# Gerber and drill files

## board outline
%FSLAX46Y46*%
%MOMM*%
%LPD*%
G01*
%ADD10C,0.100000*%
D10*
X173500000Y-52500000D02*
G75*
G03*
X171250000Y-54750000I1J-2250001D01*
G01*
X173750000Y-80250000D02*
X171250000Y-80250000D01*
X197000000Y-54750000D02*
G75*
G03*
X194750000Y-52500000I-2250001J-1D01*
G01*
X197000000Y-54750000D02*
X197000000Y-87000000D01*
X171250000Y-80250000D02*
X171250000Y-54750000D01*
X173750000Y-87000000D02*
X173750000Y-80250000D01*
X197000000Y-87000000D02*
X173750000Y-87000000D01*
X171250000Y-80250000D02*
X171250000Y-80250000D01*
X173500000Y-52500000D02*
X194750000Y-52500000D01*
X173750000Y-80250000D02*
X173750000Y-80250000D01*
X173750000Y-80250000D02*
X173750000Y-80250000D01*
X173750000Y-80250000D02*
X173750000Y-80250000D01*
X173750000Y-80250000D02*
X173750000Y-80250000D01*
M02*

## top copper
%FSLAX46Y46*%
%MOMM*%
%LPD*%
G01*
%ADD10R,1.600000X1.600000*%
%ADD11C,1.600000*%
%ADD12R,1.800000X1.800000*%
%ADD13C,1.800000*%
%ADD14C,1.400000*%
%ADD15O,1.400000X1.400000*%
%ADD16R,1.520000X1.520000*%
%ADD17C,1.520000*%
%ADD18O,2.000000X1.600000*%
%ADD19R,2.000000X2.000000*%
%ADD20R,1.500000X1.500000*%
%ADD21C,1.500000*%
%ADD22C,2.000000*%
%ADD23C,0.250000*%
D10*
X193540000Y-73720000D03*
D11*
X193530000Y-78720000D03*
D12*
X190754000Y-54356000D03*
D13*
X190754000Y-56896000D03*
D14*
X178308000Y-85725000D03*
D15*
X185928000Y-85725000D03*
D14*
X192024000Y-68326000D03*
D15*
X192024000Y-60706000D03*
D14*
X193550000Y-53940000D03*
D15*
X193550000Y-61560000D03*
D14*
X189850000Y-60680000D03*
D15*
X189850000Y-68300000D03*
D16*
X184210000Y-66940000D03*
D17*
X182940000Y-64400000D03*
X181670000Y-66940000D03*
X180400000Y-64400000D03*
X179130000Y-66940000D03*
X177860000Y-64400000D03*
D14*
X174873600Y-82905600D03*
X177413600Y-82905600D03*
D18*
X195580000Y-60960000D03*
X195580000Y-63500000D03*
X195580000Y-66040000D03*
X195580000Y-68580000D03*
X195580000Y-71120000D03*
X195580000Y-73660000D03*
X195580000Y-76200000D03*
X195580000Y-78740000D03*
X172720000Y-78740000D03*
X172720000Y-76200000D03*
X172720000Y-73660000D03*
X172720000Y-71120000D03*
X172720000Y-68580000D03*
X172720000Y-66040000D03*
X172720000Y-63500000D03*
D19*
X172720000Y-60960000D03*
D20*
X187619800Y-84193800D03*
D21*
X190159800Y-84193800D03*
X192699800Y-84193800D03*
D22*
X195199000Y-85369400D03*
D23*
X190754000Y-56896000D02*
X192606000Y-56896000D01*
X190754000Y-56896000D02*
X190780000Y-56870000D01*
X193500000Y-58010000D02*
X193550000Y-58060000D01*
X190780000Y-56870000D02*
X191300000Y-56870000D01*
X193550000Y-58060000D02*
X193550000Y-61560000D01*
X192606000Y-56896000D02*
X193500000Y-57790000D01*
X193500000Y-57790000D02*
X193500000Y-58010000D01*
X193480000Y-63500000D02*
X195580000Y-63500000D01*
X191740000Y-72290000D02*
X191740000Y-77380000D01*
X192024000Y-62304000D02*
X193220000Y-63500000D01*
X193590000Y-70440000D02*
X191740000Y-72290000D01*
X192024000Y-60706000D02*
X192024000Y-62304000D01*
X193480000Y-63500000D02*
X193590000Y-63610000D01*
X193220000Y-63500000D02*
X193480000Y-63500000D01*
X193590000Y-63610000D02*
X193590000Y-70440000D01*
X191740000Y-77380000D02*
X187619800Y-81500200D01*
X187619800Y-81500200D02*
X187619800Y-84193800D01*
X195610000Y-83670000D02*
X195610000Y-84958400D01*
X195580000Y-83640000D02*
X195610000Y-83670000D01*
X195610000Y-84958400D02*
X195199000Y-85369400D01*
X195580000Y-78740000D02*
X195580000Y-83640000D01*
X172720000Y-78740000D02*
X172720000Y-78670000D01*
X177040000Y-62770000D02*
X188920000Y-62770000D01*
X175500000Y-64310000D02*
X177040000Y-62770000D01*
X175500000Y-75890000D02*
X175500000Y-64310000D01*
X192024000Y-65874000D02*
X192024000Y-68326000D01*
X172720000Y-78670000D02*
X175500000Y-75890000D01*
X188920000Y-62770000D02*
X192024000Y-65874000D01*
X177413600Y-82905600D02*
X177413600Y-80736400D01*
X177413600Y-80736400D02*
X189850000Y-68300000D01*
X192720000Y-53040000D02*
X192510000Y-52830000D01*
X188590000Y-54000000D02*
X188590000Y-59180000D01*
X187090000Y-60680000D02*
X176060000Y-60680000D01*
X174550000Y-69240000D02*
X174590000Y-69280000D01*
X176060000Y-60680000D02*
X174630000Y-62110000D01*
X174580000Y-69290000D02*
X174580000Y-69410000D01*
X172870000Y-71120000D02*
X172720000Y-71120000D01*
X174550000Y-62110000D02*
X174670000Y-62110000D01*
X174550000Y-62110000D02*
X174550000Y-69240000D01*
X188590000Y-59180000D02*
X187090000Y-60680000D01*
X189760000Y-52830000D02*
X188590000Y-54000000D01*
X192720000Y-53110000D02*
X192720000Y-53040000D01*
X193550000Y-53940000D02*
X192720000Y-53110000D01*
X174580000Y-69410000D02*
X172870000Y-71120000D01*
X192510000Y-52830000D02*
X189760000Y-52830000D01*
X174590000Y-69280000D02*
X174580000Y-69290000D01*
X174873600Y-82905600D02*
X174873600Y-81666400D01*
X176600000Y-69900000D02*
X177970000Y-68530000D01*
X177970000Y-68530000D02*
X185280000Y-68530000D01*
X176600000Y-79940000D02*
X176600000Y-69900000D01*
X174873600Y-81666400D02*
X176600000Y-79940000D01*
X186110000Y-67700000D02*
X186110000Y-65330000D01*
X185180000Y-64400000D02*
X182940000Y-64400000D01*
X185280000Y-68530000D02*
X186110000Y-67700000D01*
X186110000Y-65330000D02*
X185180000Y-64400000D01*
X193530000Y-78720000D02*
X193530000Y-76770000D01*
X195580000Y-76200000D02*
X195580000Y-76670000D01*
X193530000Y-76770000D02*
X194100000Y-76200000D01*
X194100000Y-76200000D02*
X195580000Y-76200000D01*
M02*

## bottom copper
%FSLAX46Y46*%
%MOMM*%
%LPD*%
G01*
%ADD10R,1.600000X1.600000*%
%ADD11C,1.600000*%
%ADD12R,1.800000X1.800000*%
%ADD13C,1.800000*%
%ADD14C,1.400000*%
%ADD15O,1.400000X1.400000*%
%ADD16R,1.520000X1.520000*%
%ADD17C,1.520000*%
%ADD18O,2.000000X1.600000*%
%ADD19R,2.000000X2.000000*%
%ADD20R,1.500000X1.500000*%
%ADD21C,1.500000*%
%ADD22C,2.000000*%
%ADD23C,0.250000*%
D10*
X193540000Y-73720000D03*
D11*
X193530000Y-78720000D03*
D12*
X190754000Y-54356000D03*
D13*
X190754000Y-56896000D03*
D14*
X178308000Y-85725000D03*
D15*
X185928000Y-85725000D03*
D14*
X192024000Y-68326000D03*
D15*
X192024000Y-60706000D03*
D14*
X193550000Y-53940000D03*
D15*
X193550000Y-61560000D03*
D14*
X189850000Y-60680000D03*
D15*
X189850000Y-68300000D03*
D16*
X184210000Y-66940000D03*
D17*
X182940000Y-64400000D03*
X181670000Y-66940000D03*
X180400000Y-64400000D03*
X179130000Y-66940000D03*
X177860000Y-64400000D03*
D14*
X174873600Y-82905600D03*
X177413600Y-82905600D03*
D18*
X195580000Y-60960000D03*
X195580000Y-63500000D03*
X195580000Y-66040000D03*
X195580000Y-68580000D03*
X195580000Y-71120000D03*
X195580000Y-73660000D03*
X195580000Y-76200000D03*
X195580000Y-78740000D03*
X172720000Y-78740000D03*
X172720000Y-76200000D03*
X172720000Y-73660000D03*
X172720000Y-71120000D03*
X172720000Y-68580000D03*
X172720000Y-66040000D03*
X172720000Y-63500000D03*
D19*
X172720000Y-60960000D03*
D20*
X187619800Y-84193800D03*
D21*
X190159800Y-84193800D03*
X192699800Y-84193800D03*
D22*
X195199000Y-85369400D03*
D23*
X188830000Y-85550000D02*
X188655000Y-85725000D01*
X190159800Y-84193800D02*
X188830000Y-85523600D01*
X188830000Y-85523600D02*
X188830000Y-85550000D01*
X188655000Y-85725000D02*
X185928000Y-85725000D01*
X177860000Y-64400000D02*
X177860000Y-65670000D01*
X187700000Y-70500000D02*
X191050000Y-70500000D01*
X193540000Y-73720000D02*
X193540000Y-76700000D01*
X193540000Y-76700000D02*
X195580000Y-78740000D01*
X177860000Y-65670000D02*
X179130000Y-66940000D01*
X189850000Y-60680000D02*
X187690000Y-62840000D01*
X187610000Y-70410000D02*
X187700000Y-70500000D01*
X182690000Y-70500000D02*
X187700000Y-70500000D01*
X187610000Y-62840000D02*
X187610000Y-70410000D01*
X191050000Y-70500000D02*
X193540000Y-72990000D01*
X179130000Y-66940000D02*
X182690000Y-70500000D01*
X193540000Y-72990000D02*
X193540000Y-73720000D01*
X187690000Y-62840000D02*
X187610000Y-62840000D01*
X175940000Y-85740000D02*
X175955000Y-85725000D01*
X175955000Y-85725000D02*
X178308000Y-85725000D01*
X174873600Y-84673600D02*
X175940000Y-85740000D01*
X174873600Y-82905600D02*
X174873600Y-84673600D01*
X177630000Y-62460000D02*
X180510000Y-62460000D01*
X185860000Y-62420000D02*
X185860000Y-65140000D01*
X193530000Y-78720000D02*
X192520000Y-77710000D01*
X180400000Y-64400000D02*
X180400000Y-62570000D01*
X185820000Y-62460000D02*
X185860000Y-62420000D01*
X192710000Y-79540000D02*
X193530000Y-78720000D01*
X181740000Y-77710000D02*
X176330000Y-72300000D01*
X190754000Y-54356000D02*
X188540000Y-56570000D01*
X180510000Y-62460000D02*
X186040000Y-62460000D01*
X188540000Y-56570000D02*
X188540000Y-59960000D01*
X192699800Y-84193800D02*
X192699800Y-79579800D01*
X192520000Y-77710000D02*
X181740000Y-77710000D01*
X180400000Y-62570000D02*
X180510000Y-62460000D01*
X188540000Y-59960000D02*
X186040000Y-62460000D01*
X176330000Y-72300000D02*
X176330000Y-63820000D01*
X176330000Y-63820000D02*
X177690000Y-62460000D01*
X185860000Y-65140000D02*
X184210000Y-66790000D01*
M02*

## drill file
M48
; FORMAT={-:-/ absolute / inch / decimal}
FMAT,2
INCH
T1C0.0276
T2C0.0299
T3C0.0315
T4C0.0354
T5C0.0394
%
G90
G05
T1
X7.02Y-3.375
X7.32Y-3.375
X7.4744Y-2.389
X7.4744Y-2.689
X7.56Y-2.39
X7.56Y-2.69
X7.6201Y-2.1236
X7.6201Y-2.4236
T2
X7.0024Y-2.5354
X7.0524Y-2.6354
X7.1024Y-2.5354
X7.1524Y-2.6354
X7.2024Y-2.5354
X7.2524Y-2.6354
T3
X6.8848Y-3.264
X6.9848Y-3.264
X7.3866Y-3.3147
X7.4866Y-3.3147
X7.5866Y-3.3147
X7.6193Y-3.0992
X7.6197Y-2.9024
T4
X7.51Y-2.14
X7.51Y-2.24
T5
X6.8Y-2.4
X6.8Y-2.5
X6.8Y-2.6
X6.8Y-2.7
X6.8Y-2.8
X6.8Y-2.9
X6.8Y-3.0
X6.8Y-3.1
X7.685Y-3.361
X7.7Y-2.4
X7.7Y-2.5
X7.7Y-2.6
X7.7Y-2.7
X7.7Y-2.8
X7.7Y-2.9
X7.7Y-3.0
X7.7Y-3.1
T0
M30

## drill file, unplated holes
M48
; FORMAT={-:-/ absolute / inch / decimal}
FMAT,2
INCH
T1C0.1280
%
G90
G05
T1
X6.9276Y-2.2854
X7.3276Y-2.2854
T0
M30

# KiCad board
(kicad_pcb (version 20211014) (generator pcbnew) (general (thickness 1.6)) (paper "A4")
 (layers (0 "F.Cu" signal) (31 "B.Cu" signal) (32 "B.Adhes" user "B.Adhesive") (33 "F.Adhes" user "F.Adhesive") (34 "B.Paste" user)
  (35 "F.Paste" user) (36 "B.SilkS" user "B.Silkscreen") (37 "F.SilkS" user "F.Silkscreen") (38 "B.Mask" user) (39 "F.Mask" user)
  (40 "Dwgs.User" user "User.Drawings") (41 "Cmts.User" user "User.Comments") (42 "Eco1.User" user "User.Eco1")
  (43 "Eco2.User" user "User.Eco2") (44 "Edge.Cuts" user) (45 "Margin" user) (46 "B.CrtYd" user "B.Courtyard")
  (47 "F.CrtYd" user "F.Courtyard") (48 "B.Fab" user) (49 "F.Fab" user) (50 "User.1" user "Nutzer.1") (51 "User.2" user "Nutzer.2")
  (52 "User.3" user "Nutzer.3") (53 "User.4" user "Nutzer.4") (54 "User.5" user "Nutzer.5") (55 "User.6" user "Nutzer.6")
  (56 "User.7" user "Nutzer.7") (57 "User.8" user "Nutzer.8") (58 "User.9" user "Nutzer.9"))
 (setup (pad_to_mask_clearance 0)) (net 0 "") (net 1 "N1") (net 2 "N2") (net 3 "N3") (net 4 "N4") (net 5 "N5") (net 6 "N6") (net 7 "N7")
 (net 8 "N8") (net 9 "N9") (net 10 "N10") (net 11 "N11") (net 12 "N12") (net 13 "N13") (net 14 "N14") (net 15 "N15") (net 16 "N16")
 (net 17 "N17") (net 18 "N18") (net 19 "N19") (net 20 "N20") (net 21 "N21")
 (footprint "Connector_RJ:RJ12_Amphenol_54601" (layer "F.Cu") (at 184.21 66.94 180)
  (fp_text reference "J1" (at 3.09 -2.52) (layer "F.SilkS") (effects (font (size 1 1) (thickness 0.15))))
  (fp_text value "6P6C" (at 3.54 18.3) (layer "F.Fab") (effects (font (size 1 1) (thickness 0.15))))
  (pad "" np_thru_hole circle (at -1.91 8.89 180) (size 3.25 3.25) (drill 3.25) (layers *.Cu *.Mask))
  (pad "" np_thru_hole circle (at 8.25 8.89 180) (size 3.25 3.25) (drill 3.25) (layers *.Cu *.Mask))
  (pad "1" thru_hole rect (at 0 0 180) (size 1.52 1.52) (drill 0.76) (layers *.Cu *.Mask) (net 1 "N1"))
  (pad "2" thru_hole circle (at 1.27 2.54 180) (size 1.52 1.52) (drill 0.76) (layers *.Cu *.Mask) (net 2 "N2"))
  (pad "3" thru_hole circle (at 2.54 0 180) (size 1.52 1.52) (drill 0.76) (layers *.Cu *.Mask) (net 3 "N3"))
  (pad "4" thru_hole circle (at 3.81 2.54 180) (size 1.52 1.52) (drill 0.76) (layers *.Cu *.Mask) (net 1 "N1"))
  (pad "5" thru_hole circle (at 5.08 0 180) (size 1.52 1.52) (drill 0.76) (layers *.Cu *.Mask) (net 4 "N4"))
  (pad "6" thru_hole circle (at 6.35 2.54 180) (size 1.52 1.52) (drill 0.76) (layers *.Cu *.Mask) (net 4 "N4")))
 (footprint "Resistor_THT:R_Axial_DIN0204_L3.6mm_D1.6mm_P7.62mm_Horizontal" (layer "F.Cu") (at 192.024 68.326 90)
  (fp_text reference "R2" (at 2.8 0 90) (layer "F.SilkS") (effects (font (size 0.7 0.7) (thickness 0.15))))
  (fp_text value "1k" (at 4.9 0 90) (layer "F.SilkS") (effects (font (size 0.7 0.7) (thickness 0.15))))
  (pad "1" thru_hole circle (at 0 0 90) (size 1.4 1.4) (drill 0.7) (layers *.Cu *.Mask) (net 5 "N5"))
  (pad "2" thru_hole oval (at 7.62 0 90) (size 1.4 1.4) (drill 0.7) (layers *.Cu *.Mask) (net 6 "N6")))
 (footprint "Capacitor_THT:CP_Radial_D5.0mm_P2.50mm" (layer "F.Cu") (at 193.6 74.94 -90)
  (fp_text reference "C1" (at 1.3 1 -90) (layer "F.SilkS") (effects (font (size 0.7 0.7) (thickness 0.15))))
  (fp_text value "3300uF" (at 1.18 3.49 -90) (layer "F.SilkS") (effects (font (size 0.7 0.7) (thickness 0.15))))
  (pad "1" thru_hole rect (at -1.22 0.06 270) (size 1.6 1.6) (drill 0.8) (layers *.Cu *.Mask) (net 4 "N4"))
  (pad "2" thru_hole circle (at 3.78 0.07 270) (size 1.6 1.6) (drill 0.8) (layers *.Cu *.Mask) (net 1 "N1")))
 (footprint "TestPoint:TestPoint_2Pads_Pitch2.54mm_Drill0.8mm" (layer "F.Cu") (at 174.8736 82.9056)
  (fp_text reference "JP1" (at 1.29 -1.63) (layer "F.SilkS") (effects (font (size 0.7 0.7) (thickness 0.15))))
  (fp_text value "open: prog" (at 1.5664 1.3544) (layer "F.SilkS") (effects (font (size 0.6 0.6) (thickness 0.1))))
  (pad "1" thru_hole circle (at 0 0) (size 1.4 1.4) (drill 0.8) (layers *.Cu *.Mask) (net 2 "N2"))
  (pad "2" thru_hole circle (at 2.54 0) (size 1.4 1.4) (drill 0.8) (layers *.Cu *.Mask) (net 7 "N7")))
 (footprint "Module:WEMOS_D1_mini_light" (layer "F.Cu") (at 172.72 60.96)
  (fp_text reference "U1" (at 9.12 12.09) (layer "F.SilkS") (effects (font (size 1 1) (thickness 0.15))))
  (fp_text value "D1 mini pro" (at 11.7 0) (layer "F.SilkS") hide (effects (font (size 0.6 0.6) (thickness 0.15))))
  (pad "1" thru_hole rect (at 0 0) (size 2 2) (drill 1) (layers *.Cu *.Mask) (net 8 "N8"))
  (pad "2" thru_hole oval (at 0 2.54) (size 2 1.6) (drill 1) (layers *.Cu *.Mask) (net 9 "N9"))
  (pad "3" thru_hole oval (at 0 5.08) (size 2 1.6) (drill 1) (layers *.Cu *.Mask) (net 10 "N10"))
  (pad "4" thru_hole oval (at 0 7.62) (size 2 1.6) (drill 1) (layers *.Cu *.Mask) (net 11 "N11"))
  (pad "5" thru_hole oval (at 0 10.16) (size 2 1.6) (drill 1) (layers *.Cu *.Mask) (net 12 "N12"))
  (pad "6" thru_hole oval (at 0 12.7) (size 2 1.6) (drill 1) (layers *.Cu *.Mask) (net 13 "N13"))
  (pad "7" thru_hole oval (at 0 15.24) (size 2 1.6) (drill 1) (layers *.Cu *.Mask) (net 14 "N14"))
  (pad "8" thru_hole oval (at 0 17.78) (size 2 1.6) (drill 1) (layers *.Cu *.Mask) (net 5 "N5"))
  (pad "9" thru_hole oval (at 22.86 17.78) (size 2 1.6) (drill 1) (layers *.Cu *.Mask) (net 4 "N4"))
  (pad "10" thru_hole oval (at 22.86 15.24) (size 2 1.6) (drill 1) (layers *.Cu *.Mask) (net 1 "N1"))
  (pad "11" thru_hole oval (at 22.86 12.7) (size 2 1.6) (drill 1) (layers *.Cu *.Mask) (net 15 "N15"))
  (pad "12" thru_hole oval (at 22.86 10.16) (size 2 1.6) (drill 1) (layers *.Cu *.Mask) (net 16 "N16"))
  (pad "13" thru_hole oval (at 22.86 7.62) (size 2 1.6) (drill 1) (layers *.Cu *.Mask) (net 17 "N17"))
  (pad "14" thru_hole oval (at 22.86 5.08) (size 2 1.6) (drill 1) (layers *.Cu *.Mask) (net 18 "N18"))
  (pad "15" thru_hole oval (at 22.86 2.54) (size 2 1.6) (drill 1) (layers *.Cu *.Mask) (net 6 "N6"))
  (pad "16" thru_hole oval (at 22.86 0) (size 2 1.6) (drill 1) (layers *.Cu *.Mask) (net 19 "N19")))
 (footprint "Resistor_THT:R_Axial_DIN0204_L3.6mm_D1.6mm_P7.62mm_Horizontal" (layer "F.Cu") (at 193.55 53.94 -90)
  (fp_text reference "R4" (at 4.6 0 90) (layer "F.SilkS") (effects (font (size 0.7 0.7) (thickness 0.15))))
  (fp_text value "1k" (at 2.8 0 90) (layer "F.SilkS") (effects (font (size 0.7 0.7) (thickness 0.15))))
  (pad "1" thru_hole circle (at 0 0 270) (size 1.4 1.4) (drill 0.7) (layers *.Cu *.Mask) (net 12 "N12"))
  (pad "2" thru_hole oval (at 7.62 0 270) (size 1.4 1.4) (drill 0.7) (layers *.Cu *.Mask) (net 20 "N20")))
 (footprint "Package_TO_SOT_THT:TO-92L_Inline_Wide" (layer "F.Cu") (at 187.6198 84.1938)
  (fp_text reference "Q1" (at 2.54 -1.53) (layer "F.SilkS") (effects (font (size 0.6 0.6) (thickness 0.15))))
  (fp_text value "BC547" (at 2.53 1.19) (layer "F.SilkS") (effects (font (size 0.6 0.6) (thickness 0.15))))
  (pad "1" thru_hole rect (at 0 0) (size 1.5 1.5) (drill 0.8) (layers *.Cu *.Mask) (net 6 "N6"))
  (pad "2" thru_hole circle (at 2.54 0) (size 1.5 1.5) (drill 0.8) (layers *.Cu *.Mask) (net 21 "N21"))
  (pad "3" thru_hole circle (at 5.08 0) (size 1.5 1.5) (drill 0.8) (layers *.Cu *.Mask) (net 1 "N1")))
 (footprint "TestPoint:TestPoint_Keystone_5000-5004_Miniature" (layer "F.Cu") (at 195.199 85.3694)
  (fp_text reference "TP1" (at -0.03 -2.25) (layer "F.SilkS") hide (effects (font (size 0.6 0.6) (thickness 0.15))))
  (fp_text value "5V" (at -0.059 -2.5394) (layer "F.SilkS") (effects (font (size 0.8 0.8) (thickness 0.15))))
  (pad "1" thru_hole circle (at 0 0) (size 2 2) (drill 1) (layers *.Cu *.Mask) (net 4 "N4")))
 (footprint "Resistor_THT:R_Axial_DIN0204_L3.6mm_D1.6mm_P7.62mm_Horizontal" (layer "F.Cu") (at 189.85 60.68 -90)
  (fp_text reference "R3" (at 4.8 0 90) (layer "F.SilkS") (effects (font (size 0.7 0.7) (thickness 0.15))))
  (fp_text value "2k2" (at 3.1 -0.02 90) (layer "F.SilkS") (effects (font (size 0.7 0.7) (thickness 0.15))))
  (pad "1" thru_hole circle (at 0 0 270) (size 1.4 1.4) (drill 0.7) (layers *.Cu *.Mask) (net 4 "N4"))
  (pad "2" thru_hole oval (at 7.62 0 270) (size 1.4 1.4) (drill 0.7) (layers *.Cu *.Mask) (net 7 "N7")))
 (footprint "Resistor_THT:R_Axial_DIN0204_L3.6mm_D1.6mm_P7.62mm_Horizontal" (layer "F.Cu") (at 178.308 85.725)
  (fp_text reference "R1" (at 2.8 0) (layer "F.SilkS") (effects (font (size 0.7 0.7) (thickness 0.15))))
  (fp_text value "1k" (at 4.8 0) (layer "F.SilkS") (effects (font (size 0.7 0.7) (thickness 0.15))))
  (pad "1" thru_hole circle (at 0 0) (size 1.4 1.4) (drill 0.7) (layers *.Cu *.Mask) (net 2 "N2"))
  (pad "2" thru_hole oval (at 7.62 0) (size 1.4 1.4) (drill 0.7) (layers *.Cu *.Mask) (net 21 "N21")))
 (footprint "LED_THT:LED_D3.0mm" (layer "F.Cu") (at 190.754 54.356 -90)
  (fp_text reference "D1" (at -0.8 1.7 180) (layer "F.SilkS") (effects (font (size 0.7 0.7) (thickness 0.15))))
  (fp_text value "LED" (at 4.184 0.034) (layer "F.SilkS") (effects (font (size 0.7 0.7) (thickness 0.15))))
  (pad "1" thru_hole rect (at 0 0 270) (size 1.8 1.8) (drill 0.9) (layers *.Cu *.Mask) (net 1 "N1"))
  (pad "2" thru_hole circle (at 2.54 0 270) (size 1.8 1.8) (drill 0.9) (layers *.Cu *.Mask) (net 20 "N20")))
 (gr_arc (start 171.25 54.75) (mid 171.90901 53.15901) (end 173.5 52.5) (layer "Edge.Cuts") (width 0.1))
 (gr_line (start 173.75 80.25) (end 171.25 80.25) (layer "Edge.Cuts") (width 0.1))
 (gr_arc (start 194.75 52.5) (mid 196.34099 53.15901) (end 197 54.75) (layer "Edge.Cuts") (width 0.1))
 (gr_line (start 197 54.75) (end 197 87) (layer "Edge.Cuts") (width 0.1))
 (gr_line (start 171.25 80.25) (end 171.25 54.75) (layer "Edge.Cuts") (width 0.1))
 (gr_line (start 173.75 87) (end 173.75 80.25) (layer "Edge.Cuts") (width 0.1))
 (gr_line (start 197 87) (end 173.75 87) (layer "Edge.Cuts") (width 0.1))
 (gr_line (start 171.25 80.25) (end 171.25 80.25) (layer "Edge.Cuts") (width 0.1))
 (gr_line (start 173.5 52.5) (end 194.75 52.5) (layer "Edge.Cuts") (width 0.1))
 (gr_rect (start 173.75 80.25) (end 173.75 80.25) (layer "Edge.Cuts") (width 0.1) (fill none))
 (segment (start 190.754 56.896) (end 192.606 56.896) (width 0.25) (layer "F.Cu") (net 20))
 (segment (start 190.754 56.896) (end 190.78 56.87) (width 0.25) (layer "F.Cu") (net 20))
 (segment (start 193.5 58.01) (end 193.55 58.06) (width 0.25) (layer "F.Cu") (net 20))
 (segment (start 190.78 56.87) (end 191.3 56.87) (width 0.25) (layer "F.Cu") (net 20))
 (segment (start 193.55 58.06) (end 193.55 61.56) (width 0.25) (layer "F.Cu") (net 20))
 (segment (start 192.606 56.896) (end 193.5 57.79) (width 0.25) (layer "F.Cu") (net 20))
 (segment (start 193.5 57.79) (end 193.5 58.01) (width 0.25) (layer "F.Cu") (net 20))
 (segment (start 188.83 85.55) (end 188.655 85.725) (width 0.25) (layer "B.Cu") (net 21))
 (segment (start 190.1598 84.1938) (end 188.83 85.5236) (width 0.25) (layer "B.Cu") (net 21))
 (segment (start 188.83 85.5236) (end 188.83 85.55) (width 0.25) (layer "B.Cu") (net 21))
 (segment (start 188.655 85.725) (end 185.928 85.725) (width 0.25) (layer "B.Cu") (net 21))
 (segment (start 193.48 63.5) (end 195.58 63.5) (width 0.25) (layer "F.Cu") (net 6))
 (segment (start 191.74 72.29) (end 191.74 77.38) (width 0.25) (layer "F.Cu") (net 6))
 (segment (start 192.024 62.304) (end 193.22 63.5) (width 0.25) (layer "F.Cu") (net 6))
 (segment (start 193.59 70.44) (end 191.74 72.29) (width 0.25) (layer "F.Cu") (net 6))
 (segment (start 192.024 60.706) (end 192.024 62.304) (width 0.25) (layer "F.Cu") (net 6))
 (segment (start 193.48 63.5) (end 193.59 63.61) (width 0.25) (layer "F.Cu") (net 6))
 (segment (start 193.22 63.5) (end 193.48 63.5) (width 0.25) (layer "F.Cu") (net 6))
 (segment (start 193.59 63.61) (end 193.59 70.44) (width 0.25) (layer "F.Cu") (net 6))
 (segment (start 191.74 77.38) (end 187.6198 81.5002) (width 0.25) (layer "F.Cu") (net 6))
 (segment (start 187.6198 81.5002) (end 187.6198 84.1938) (width 0.25) (layer "F.Cu") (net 6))
 (segment (start 195.61 83.67) (end 195.61 84.9584) (width 0.25) (layer "F.Cu") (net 4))
 (segment (start 195.58 83.64) (end 195.61 83.67) (width 0.25) (layer "F.Cu") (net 4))
 (segment (start 195.61 84.9584) (end 195.199 85.3694) (width 0.25) (layer "F.Cu") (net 4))
 (segment (start 195.58 78.74) (end 195.58 83.64) (width 0.25) (layer "F.Cu") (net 4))
 (segment (start 177.86 64.4) (end 177.86 65.67) (width 0.25) (layer "B.Cu") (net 4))
 (segment (start 187.7 70.5) (end 191.05 70.5) (width 0.25) (layer "B.Cu") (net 4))
 (segment (start 193.54 73.72) (end 193.54 76.7) (width 0.25) (layer "B.Cu") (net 4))
 (segment (start 193.54 76.7) (end 195.58 78.74) (width 0.25) (layer "B.Cu") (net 4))
 (segment (start 177.86 65.67) (end 179.13 66.94) (width 0.25) (layer "B.Cu") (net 4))
 (segment (start 189.85 60.68) (end 187.69 62.84) (width 0.25) (layer "B.Cu") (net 4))
 (segment (start 187.61 70.41) (end 187.7 70.5) (width 0.25) (layer "B.Cu") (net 4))
 (segment (start 182.69 70.5) (end 187.7 70.5) (width 0.25) (layer "B.Cu") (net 4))
 (segment (start 187.61 62.84) (end 187.61 70.41) (width 0.25) (layer "B.Cu") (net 4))
 (segment (start 191.05 70.5) (end 193.54 72.99) (width 0.25) (layer "B.Cu") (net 4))
 (segment (start 179.13 66.94) (end 182.69 70.5) (width 0.25) (layer "B.Cu") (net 4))
 (segment (start 193.54 72.99) (end 193.54 73.72) (width 0.25) (layer "B.Cu") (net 4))
 (segment (start 187.69 62.84) (end 187.61 62.84) (width 0.25) (layer "B.Cu") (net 4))
 (segment (start 172.72 78.74) (end 172.72 78.67) (width 0.25) (layer "F.Cu") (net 5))
 (segment (start 177.04 62.77) (end 188.92 62.77) (width 0.25) (layer "F.Cu") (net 5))
 (segment (start 175.5 64.31) (end 177.04 62.77) (width 0.25) (layer "F.Cu") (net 5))
 (segment (start 175.5 75.89) (end 175.5 64.31) (width 0.25) (layer "F.Cu") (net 5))
 (segment (start 192.024 65.874) (end 192.024 68.326) (width 0.25) (layer "F.Cu") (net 5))
 (segment (start 172.72 78.67) (end 175.5 75.89) (width 0.25) (layer "F.Cu") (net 5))
 (segment (start 188.92 62.77) (end 192.024 65.874) (width 0.25) (layer "F.Cu") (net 5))
 (segment (start 177.4136 82.9056) (end 177.4136 80.7364) (width 0.25) (layer "F.Cu") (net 7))
 (segment (start 177.4136 80.7364) (end 189.85 68.3) (width 0.25) (layer "F.Cu") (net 7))
 (segment (start 192.72 53.04) (end 192.51 52.83) (width 0.25) (layer "F.Cu") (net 12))
 (segment (start 188.59 54) (end 188.59 59.18) (width 0.25) (layer "F.Cu") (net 12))
 (segment (start 187.09 60.68) (end 176.06 60.68) (width 0.25) (layer "F.Cu") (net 12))
 (segment (start 174.55 69.24) (end 174.59 69.28) (width 0.25) (layer "F.Cu") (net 12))
 (segment (start 176.06 60.68) (end 174.63 62.11) (width 0.25) (layer "F.Cu") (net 12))
 (segment (start 174.58 69.29) (end 174.58 69.41) (width 0.25) (layer "F.Cu") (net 12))
 (segment (start 172.87 71.12) (end 172.72 71.12) (width 0.25) (layer "F.Cu") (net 12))
 (segment (start 174.55 62.11) (end 174.67 62.11) (width 0.25) (layer "F.Cu") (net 12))
 (segment (start 174.55 62.11) (end 174.55 69.24) (width 0.25) (layer "F.Cu") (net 12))
 (segment (start 188.59 59.18) (end 187.09 60.68) (width 0.25) (layer "F.Cu") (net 12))
 (segment (start 189.76 52.83) (end 188.59 54) (width 0.25) (layer "F.Cu") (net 12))
 (segment (start 192.72 53.11) (end 192.72 53.04) (width 0.25) (layer "F.Cu") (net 12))
 (segment (start 193.55 53.94) (end 192.72 53.11) (width 0.25) (layer "F.Cu") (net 12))
 (segment (start 174.58 69.41) (end 172.87 71.12) (width 0.25) (layer "F.Cu") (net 12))
 (segment (start 192.51 52.83) (end 189.76 52.83) (width 0.25) (layer "F.Cu") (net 12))
 (segment (start 174.59 69.28) (end 174.58 69.29) (width 0.25) (layer "F.Cu") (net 12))
 (segment (start 174.8736 82.9056) (end 174.8736 81.6664) (width 0.25) (layer "F.Cu") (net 2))
 (segment (start 176.6 69.9) (end 177.97 68.53) (width 0.25) (layer "F.Cu") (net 2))
 (segment (start 177.97 68.53) (end 185.28 68.53) (width 0.25) (layer "F.Cu") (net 2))
 (segment (start 176.6 79.94) (end 176.6 69.9) (width 0.25) (layer "F.Cu") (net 2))
 (segment (start 174.8736 81.6664) (end 176.6 79.94) (width 0.25) (layer "F.Cu") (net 2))
 (segment (start 186.11 67.7) (end 186.11 65.33) (width 0.25) (layer "F.Cu") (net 2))
 (segment (start 185.18 64.4) (end 182.94 64.4) (width 0.25) (layer "F.Cu") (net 2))
 (segment (start 185.28 68.53) (end 186.11 67.7) (width 0.25) (layer "F.Cu") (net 2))
 (segment (start 186.11 65.33) (end 185.18 64.4) (width 0.25) (layer "F.Cu") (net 2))
 (segment (start 175.94 85.74) (end 175.955 85.725) (width 0.25) (layer "B.Cu") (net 2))
 (segment (start 175.955 85.725) (end 178.308 85.725) (width 0.25) (layer "B.Cu") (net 2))
 (segment (start 174.8736 84.6736) (end 175.94 85.74) (width 0.25) (layer "B.Cu") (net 2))
 (segment (start 174.8736 82.9056) (end 174.8736 84.6736) (width 0.25) (layer "B.Cu") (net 2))
 (segment (start 193.53 78.72) (end 193.53 76.77) (width 0.25) (layer "F.Cu") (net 1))
 (segment (start 195.58 76.2) (end 195.58 76.67) (width 0.25) (layer "F.Cu") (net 1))
 (segment (start 193.53 76.77) (end 194.1 76.2) (width 0.25) (layer "F.Cu") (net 1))
 (segment (start 194.1 76.2) (end 195.58 76.2) (width 0.25) (layer "F.Cu") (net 1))
 (segment (start 177.63 62.46) (end 180.51 62.46) (width 0.25) (layer "B.Cu") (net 1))
 (segment (start 185.86 62.42) (end 185.86 65.14) (width 0.25) (layer "B.Cu") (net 1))
 (segment (start 193.53 78.72) (end 192.52 77.71) (width 0.25) (layer "B.Cu") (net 1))
 (segment (start 180.4 64.4) (end 180.4 62.57) (width 0.25) (layer "B.Cu") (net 1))
 (segment (start 185.82 62.46) (end 185.86 62.42) (width 0.25) (layer "B.Cu") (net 1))
 (segment (start 192.71 79.54) (end 193.53 78.72) (width 0.25) (layer "B.Cu") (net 1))
 (segment (start 181.74 77.71) (end 176.33 72.3) (width 0.25) (layer "B.Cu") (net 1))
 (segment (start 190.754 54.356) (end 188.54 56.57) (width 0.25) (layer "B.Cu") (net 1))
 (segment (start 180.51 62.46) (end 186.04 62.46) (width 0.25) (layer "B.Cu") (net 1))
 (segment (start 188.54 56.57) (end 188.54 59.96) (width 0.25) (layer "B.Cu") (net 1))
 (segment (start 192.6998 84.1938) (end 192.6998 79.5798) (width 0.25) (layer "B.Cu") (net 1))
 (segment (start 192.52 77.71) (end 181.74 77.71) (width 0.25) (layer "B.Cu") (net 1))
 (segment (start 180.4 62.57) (end 180.51 62.46) (width 0.25) (layer "B.Cu") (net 1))
 (segment (start 188.54 59.96) (end 186.04 62.46) (width 0.25) (layer "B.Cu") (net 1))
 (segment (start 176.33 72.3) (end 176.33 63.82) (width 0.25) (layer "B.Cu") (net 1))
 (segment (start 176.33 63.82) (end 177.69 62.46) (width 0.25) (layer "B.Cu") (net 1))
 (segment (start 185.86 65.14) (end 184.21 66.79) (width 0.25) (layer "B.Cu") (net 1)))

